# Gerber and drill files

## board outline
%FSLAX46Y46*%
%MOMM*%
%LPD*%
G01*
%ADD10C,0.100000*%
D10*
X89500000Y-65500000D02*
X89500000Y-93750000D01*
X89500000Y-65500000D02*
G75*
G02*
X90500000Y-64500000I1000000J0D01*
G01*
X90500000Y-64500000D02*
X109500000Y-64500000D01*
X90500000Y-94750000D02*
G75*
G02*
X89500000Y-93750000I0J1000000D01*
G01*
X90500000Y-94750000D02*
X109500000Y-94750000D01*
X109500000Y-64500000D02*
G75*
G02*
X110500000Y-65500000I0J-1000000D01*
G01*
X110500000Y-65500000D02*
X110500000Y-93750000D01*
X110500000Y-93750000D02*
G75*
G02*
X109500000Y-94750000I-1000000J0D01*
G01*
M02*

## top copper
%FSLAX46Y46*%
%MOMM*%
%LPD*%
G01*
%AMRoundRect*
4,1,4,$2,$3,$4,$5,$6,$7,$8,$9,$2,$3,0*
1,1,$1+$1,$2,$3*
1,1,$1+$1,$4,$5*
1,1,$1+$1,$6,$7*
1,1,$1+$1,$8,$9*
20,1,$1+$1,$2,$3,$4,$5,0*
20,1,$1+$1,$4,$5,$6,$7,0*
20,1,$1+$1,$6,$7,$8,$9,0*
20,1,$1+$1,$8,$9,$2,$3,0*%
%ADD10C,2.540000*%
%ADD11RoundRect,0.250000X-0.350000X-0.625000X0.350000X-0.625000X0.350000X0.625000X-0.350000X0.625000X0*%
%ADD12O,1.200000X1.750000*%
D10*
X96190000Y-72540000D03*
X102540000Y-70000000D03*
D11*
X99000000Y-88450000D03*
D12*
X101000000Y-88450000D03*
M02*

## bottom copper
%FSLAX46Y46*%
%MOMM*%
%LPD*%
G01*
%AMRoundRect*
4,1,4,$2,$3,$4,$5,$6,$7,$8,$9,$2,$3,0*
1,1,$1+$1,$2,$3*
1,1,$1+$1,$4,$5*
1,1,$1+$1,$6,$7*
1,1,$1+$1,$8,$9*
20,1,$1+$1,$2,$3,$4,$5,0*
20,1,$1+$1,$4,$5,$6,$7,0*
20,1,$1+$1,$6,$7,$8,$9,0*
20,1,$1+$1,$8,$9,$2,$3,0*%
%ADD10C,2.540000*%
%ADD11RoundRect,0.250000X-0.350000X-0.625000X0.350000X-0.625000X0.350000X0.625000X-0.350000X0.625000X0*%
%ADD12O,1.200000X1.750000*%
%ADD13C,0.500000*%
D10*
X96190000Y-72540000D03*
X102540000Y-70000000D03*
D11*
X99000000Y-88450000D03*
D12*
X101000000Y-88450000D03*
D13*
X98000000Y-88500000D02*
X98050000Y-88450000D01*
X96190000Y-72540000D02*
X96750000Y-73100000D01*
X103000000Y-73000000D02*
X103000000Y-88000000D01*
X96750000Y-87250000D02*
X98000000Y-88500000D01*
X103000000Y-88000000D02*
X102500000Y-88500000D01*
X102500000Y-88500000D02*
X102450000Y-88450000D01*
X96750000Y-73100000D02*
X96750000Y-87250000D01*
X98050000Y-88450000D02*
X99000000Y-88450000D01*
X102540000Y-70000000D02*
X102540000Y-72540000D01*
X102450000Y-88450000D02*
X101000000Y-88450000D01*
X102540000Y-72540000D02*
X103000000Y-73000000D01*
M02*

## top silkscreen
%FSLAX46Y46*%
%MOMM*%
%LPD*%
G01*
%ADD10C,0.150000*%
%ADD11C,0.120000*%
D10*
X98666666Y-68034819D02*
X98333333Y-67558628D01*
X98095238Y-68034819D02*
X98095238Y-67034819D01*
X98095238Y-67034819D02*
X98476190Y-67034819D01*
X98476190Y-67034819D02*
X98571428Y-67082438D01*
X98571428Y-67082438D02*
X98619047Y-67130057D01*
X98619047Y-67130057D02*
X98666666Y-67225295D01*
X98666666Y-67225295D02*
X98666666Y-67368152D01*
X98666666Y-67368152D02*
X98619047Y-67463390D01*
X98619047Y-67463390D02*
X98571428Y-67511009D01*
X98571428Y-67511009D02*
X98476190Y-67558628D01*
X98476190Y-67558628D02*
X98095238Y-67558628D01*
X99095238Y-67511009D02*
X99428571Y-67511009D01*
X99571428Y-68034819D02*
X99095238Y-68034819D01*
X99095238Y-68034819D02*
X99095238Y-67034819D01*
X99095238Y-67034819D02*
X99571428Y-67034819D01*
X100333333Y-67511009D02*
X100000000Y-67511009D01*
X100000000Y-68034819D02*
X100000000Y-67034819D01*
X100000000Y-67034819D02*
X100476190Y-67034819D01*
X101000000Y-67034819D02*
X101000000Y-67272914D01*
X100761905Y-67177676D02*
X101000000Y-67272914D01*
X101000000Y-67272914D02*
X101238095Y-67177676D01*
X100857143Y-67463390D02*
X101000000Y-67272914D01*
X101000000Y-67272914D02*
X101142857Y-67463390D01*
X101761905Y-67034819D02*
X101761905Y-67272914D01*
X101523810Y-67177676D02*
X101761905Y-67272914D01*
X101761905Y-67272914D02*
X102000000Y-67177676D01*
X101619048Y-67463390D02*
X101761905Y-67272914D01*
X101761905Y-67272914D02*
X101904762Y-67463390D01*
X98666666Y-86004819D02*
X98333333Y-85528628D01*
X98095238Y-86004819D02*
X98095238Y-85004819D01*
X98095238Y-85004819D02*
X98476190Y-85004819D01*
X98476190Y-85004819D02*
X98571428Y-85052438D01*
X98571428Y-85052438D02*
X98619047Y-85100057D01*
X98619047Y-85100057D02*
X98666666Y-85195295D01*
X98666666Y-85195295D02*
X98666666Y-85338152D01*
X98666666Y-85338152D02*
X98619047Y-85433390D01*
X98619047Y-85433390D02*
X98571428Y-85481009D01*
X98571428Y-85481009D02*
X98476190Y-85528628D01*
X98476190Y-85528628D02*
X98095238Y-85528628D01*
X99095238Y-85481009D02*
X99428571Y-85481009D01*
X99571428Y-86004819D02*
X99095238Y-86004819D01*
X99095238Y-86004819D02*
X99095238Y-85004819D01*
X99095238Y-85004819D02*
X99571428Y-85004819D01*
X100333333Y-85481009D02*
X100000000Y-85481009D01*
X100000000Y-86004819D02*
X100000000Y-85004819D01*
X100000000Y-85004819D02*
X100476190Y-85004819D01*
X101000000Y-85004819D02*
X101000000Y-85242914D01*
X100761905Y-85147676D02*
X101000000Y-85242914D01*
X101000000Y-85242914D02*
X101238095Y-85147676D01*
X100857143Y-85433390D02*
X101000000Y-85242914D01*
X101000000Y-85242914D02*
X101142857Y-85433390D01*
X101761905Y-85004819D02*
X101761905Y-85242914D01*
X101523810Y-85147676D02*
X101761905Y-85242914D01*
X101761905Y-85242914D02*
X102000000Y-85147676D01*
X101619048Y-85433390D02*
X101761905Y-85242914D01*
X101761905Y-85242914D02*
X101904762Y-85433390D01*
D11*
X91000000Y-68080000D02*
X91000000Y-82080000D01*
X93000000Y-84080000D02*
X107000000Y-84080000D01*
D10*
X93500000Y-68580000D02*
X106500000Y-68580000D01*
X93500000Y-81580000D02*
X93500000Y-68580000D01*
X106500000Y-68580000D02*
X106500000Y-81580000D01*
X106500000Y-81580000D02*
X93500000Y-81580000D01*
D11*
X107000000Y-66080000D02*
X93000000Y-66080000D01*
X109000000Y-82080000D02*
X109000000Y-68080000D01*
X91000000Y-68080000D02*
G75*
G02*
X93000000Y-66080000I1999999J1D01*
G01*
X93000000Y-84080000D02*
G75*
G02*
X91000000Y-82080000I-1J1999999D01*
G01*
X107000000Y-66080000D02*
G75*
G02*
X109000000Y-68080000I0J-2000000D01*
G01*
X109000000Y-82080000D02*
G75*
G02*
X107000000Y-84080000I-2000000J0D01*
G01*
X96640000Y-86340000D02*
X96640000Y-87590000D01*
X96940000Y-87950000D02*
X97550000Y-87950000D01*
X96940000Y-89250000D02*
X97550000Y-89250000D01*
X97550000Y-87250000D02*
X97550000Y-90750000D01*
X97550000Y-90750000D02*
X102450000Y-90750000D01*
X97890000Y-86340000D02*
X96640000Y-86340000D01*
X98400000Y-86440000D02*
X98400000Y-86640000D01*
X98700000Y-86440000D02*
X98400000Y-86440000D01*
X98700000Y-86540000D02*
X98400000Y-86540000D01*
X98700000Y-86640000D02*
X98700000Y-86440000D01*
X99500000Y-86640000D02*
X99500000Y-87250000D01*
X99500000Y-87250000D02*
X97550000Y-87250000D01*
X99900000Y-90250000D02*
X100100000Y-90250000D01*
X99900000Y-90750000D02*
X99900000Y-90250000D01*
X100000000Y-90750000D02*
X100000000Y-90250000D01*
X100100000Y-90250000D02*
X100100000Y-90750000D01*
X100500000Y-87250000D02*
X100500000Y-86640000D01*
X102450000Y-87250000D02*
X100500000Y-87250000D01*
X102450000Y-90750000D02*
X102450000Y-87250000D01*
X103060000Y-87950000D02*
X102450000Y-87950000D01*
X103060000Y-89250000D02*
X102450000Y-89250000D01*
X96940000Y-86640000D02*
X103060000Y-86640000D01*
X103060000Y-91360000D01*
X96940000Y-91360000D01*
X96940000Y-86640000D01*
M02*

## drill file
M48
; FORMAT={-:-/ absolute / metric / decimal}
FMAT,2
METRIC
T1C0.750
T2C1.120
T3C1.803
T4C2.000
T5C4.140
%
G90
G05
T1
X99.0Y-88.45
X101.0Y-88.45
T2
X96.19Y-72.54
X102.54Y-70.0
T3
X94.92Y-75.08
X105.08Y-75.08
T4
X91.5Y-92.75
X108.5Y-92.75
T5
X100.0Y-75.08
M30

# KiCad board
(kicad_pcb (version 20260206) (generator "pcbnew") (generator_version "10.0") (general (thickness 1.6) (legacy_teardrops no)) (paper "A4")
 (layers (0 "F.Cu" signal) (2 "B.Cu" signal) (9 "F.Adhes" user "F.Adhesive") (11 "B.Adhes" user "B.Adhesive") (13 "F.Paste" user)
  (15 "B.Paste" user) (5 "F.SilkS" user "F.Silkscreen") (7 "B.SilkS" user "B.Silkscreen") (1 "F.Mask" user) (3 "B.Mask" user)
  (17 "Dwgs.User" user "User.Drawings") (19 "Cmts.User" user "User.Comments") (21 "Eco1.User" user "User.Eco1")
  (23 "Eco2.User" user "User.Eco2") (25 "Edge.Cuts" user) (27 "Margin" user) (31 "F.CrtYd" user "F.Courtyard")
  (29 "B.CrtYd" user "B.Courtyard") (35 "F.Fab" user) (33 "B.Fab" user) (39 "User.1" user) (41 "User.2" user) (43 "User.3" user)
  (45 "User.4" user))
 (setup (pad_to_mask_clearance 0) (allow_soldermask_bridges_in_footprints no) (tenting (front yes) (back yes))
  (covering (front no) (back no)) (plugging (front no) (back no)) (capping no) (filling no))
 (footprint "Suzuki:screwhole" (layer "F.Cu") (at 108.75 92.75)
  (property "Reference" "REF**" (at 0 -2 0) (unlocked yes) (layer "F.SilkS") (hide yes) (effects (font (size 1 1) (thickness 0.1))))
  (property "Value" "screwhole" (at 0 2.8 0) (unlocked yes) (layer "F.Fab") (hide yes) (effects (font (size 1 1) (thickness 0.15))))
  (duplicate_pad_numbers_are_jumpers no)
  (pad "" np_thru_hole circle (at -0.25 0) (size 2 2) (drill 2) (layers "*.Cu" "*.Mask")))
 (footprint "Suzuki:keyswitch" (layer "F.Cu") (at 100 75.08)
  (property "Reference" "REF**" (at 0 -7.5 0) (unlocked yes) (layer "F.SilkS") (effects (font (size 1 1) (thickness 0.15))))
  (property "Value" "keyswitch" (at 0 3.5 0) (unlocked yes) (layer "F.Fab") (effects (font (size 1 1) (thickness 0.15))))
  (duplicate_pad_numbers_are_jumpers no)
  (fp_line (start -9 -7) (end -9 7) (stroke (width 0.12) (type default)) (layer "F.SilkS"))
  (fp_line (start -7 9) (end 7 9) (stroke (width 0.12) (type default)) (layer "F.SilkS"))
  (fp_line (start -6.5 -6.5) (end 6.5 -6.5) (stroke (width 0.15) (type solid)) (layer "F.SilkS"))
  (fp_line (start -6.5 6.5) (end -6.5 -6.5) (stroke (width 0.15) (type solid)) (layer "F.SilkS"))
  (fp_line (start 6.5 -6.5) (end 6.5 6.5) (stroke (width 0.15) (type solid)) (layer "F.SilkS"))
  (fp_line (start 6.5 6.5) (end -6.5 6.5) (stroke (width 0.15) (type solid)) (layer "F.SilkS"))
  (fp_line (start 7 -9) (end -7 -9) (stroke (width 0.12) (type default)) (layer "F.SilkS"))
  (fp_line (start 9 7) (end 9 -7) (stroke (width 0.12) (type default)) (layer "F.SilkS"))
  (fp_arc (start -9 -7) (mid -8.414214 -8.414214) (end -7 -9) (stroke (width 0.12) (type default)) (layer "F.SilkS"))
  (fp_arc (start -7 9) (mid -8.414214 8.414214) (end -9 7) (stroke (width 0.12) (type default)) (layer "F.SilkS"))
  (fp_arc (start 7 -9) (mid 8.414214 -8.414214) (end 9 -7) (stroke (width 0.12) (type default)) (layer "F.SilkS"))
  (fp_arc (start 9 7) (mid 8.414214 8.414214) (end 7 9) (stroke (width 0.12) (type default)) (layer "F.SilkS"))
  (pad "" np_thru_hole circle (at -5.08 0) (size 1.8034 1.8034) (drill 1.8034) (layers "*.Cu" "*.Mask"))
  (pad "" np_thru_hole circle (at 0 0) (size 4.1402 4.1402) (drill 4.1402) (layers "*.Cu" "*.Mask"))
  (pad "" np_thru_hole circle (at 5.08 0) (size 1.8034 1.8034) (drill 1.8034) (layers "*.Cu" "*.Mask"))
  (pad "1" thru_hole circle (at -3.81 -2.54) (size 2.54 2.54) (drill 1.12) (layers "*.Cu" "*.Mask") (remove_unused_layers no))
  (pad "2" thru_hole circle (at 2.54 -5.08) (size 2.54 2.54) (drill 1.12) (layers "*.Cu" "*.Mask") (remove_unused_layers no)))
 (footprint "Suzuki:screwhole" (layer "F.Cu") (at 91.5 92.75)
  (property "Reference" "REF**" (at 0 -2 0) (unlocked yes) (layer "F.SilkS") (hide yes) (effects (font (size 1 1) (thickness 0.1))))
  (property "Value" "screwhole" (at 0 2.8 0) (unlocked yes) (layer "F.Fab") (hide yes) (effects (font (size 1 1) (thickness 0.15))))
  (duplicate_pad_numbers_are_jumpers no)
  (pad "" np_thru_hole circle (at 0 0) (size 2 2) (drill 2) (layers "*.Cu" "*.Mask")))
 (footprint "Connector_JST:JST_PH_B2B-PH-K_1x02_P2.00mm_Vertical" (layer "F.Cu") (at 99 88.45)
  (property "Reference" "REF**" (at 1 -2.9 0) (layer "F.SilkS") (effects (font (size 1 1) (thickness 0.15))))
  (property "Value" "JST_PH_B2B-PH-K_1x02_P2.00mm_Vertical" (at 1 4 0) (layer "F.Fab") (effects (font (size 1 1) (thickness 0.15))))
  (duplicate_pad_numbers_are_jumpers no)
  (fp_line (start -2.36 -2.11) (end -2.36 -0.86) (stroke (width 0.12) (type solid)) (layer "F.SilkS"))
  (fp_line (start -2.06 -0.5) (end -1.45 -0.5) (stroke (width 0.12) (type solid)) (layer "F.SilkS"))
  (fp_line (start -2.06 0.8) (end -1.45 0.8) (stroke (width 0.12) (type solid)) (layer "F.SilkS"))
  (fp_line (start -1.45 -1.2) (end -1.45 2.3) (stroke (width 0.12) (type solid)) (layer "F.SilkS"))
  (fp_line (start -1.45 2.3) (end 3.45 2.3) (stroke (width 0.12) (type solid)) (layer "F.SilkS"))
  (fp_line (start -1.11 -2.11) (end -2.36 -2.11) (stroke (width 0.12) (type solid)) (layer "F.SilkS"))
  (fp_line (start -0.6 -2.01) (end -0.6 -1.81) (stroke (width 0.12) (type solid)) (layer "F.SilkS"))
  (fp_line (start -0.3 -2.01) (end -0.6 -2.01) (stroke (width 0.12) (type solid)) (layer "F.SilkS"))
  (fp_line (start -0.3 -1.91) (end -0.6 -1.91) (stroke (width 0.12) (type solid)) (layer "F.SilkS"))
  (fp_line (start -0.3 -1.81) (end -0.3 -2.01) (stroke (width 0.12) (type solid)) (layer "F.SilkS"))
  (fp_line (start 0.5 -1.81) (end 0.5 -1.2) (stroke (width 0.12) (type solid)) (layer "F.SilkS"))
  (fp_line (start 0.5 -1.2) (end -1.45 -1.2) (stroke (width 0.12) (type solid)) (layer "F.SilkS"))
  (fp_line (start 0.9 1.8) (end 1.1 1.8) (stroke (width 0.12) (type solid)) (layer "F.SilkS"))
  (fp_line (start 0.9 2.3) (end 0.9 1.8) (stroke (width 0.12) (type solid)) (layer "F.SilkS"))
  (fp_line (start 1 2.3) (end 1 1.8) (stroke (width 0.12) (type solid)) (layer "F.SilkS"))
  (fp_line (start 1.1 1.8) (end 1.1 2.3) (stroke (width 0.12) (type solid)) (layer "F.SilkS"))
  (fp_line (start 1.5 -1.2) (end 1.5 -1.81) (stroke (width 0.12) (type solid)) (layer "F.SilkS"))
  (fp_line (start 3.45 -1.2) (end 1.5 -1.2) (stroke (width 0.12) (type solid)) (layer "F.SilkS"))
  (fp_line (start 3.45 2.3) (end 3.45 -1.2) (stroke (width 0.12) (type solid)) (layer "F.SilkS"))
  (fp_line (start 4.06 -0.5) (end 3.45 -0.5) (stroke (width 0.12) (type solid)) (layer "F.SilkS"))
  (fp_line (start 4.06 0.8) (end 3.45 0.8) (stroke (width 0.12) (type solid)) (layer "F.SilkS"))
  (fp_rect (start -2.06 -1.81) (end 4.06 2.91) (stroke (width 0.12) (type solid)) (fill no) (layer "F.SilkS"))
  (pad "1" thru_hole roundrect (at 0 0) (size 1.2 1.75) (drill 0.75) (layers "*.Cu" "*.Mask") (remove_unused_layers no)
   (roundrect_rratio 0.208333))
  (pad "2" thru_hole oval (at 2 0) (size 1.2 1.75) (drill 0.75) (layers "*.Cu" "*.Mask") (remove_unused_layers no)))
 (gr_line (start 89.5 65.5) (end 89.5 93.75) (stroke (width 0.1) (type solid)) (layer "Edge.Cuts"))
 (gr_arc (start 89.5 65.5) (mid 89.792893 64.792893) (end 90.5 64.5) (stroke (width 0.1) (type default)) (layer "Edge.Cuts"))
 (gr_line (start 90.5 64.5) (end 109.5 64.5) (stroke (width 0.1) (type solid)) (layer "Edge.Cuts"))
 (gr_arc (start 90.5 94.75) (mid 89.792893 94.457107) (end 89.5 93.75) (stroke (width 0.1) (type default)) (layer "Edge.Cuts"))
 (gr_line (start 90.5 94.75) (end 109.5 94.75) (stroke (width 0.1) (type solid)) (layer "Edge.Cuts"))
 (gr_arc (start 109.5 64.5) (mid 110.207107 64.792893) (end 110.5 65.5) (stroke (width 0.1) (type default)) (layer "Edge.Cuts"))
 (gr_line (start 110.5 65.5) (end 110.5 93.75) (stroke (width 0.1) (type solid)) (layer "Edge.Cuts"))
 (gr_arc (start 110.5 93.75) (mid 110.207107 94.457107) (end 109.5 94.75) (stroke (width 0.1) (type default)) (layer "Edge.Cuts"))
 (segment (start 98 88.5) (end 98.05 88.45) (width 0.5) (layer "B.Cu") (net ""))
 (segment (start 96.19 72.54) (end 96.75 73.1) (width 0.5) (layer "B.Cu") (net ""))
 (segment (start 103 73) (end 103 88) (width 0.5) (layer "B.Cu") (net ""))
 (segment (start 96.75 87.25) (end 98 88.5) (width 0.5) (layer "B.Cu") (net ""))
 (segment (start 103 88) (end 102.5 88.5) (width 0.5) (layer "B.Cu") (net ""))
 (segment (start 102.5 88.5) (end 102.45 88.45) (width 0.5) (layer "B.Cu") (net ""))
 (segment (start 96.75 73.1) (end 96.75 87.25) (width 0.5) (layer "B.Cu") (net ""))
 (segment (start 98.05 88.45) (end 99 88.45) (width 0.5) (layer "B.Cu") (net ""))
 (segment (start 102.54 70) (end 102.54 72.54) (width 0.5) (layer "B.Cu") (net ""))
 (segment (start 102.45 88.45) (end 101 88.45) (width 0.5) (layer "B.Cu") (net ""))
 (segment (start 102.54 72.54) (end 103 73) (width 0.5) (layer "B.Cu") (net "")))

